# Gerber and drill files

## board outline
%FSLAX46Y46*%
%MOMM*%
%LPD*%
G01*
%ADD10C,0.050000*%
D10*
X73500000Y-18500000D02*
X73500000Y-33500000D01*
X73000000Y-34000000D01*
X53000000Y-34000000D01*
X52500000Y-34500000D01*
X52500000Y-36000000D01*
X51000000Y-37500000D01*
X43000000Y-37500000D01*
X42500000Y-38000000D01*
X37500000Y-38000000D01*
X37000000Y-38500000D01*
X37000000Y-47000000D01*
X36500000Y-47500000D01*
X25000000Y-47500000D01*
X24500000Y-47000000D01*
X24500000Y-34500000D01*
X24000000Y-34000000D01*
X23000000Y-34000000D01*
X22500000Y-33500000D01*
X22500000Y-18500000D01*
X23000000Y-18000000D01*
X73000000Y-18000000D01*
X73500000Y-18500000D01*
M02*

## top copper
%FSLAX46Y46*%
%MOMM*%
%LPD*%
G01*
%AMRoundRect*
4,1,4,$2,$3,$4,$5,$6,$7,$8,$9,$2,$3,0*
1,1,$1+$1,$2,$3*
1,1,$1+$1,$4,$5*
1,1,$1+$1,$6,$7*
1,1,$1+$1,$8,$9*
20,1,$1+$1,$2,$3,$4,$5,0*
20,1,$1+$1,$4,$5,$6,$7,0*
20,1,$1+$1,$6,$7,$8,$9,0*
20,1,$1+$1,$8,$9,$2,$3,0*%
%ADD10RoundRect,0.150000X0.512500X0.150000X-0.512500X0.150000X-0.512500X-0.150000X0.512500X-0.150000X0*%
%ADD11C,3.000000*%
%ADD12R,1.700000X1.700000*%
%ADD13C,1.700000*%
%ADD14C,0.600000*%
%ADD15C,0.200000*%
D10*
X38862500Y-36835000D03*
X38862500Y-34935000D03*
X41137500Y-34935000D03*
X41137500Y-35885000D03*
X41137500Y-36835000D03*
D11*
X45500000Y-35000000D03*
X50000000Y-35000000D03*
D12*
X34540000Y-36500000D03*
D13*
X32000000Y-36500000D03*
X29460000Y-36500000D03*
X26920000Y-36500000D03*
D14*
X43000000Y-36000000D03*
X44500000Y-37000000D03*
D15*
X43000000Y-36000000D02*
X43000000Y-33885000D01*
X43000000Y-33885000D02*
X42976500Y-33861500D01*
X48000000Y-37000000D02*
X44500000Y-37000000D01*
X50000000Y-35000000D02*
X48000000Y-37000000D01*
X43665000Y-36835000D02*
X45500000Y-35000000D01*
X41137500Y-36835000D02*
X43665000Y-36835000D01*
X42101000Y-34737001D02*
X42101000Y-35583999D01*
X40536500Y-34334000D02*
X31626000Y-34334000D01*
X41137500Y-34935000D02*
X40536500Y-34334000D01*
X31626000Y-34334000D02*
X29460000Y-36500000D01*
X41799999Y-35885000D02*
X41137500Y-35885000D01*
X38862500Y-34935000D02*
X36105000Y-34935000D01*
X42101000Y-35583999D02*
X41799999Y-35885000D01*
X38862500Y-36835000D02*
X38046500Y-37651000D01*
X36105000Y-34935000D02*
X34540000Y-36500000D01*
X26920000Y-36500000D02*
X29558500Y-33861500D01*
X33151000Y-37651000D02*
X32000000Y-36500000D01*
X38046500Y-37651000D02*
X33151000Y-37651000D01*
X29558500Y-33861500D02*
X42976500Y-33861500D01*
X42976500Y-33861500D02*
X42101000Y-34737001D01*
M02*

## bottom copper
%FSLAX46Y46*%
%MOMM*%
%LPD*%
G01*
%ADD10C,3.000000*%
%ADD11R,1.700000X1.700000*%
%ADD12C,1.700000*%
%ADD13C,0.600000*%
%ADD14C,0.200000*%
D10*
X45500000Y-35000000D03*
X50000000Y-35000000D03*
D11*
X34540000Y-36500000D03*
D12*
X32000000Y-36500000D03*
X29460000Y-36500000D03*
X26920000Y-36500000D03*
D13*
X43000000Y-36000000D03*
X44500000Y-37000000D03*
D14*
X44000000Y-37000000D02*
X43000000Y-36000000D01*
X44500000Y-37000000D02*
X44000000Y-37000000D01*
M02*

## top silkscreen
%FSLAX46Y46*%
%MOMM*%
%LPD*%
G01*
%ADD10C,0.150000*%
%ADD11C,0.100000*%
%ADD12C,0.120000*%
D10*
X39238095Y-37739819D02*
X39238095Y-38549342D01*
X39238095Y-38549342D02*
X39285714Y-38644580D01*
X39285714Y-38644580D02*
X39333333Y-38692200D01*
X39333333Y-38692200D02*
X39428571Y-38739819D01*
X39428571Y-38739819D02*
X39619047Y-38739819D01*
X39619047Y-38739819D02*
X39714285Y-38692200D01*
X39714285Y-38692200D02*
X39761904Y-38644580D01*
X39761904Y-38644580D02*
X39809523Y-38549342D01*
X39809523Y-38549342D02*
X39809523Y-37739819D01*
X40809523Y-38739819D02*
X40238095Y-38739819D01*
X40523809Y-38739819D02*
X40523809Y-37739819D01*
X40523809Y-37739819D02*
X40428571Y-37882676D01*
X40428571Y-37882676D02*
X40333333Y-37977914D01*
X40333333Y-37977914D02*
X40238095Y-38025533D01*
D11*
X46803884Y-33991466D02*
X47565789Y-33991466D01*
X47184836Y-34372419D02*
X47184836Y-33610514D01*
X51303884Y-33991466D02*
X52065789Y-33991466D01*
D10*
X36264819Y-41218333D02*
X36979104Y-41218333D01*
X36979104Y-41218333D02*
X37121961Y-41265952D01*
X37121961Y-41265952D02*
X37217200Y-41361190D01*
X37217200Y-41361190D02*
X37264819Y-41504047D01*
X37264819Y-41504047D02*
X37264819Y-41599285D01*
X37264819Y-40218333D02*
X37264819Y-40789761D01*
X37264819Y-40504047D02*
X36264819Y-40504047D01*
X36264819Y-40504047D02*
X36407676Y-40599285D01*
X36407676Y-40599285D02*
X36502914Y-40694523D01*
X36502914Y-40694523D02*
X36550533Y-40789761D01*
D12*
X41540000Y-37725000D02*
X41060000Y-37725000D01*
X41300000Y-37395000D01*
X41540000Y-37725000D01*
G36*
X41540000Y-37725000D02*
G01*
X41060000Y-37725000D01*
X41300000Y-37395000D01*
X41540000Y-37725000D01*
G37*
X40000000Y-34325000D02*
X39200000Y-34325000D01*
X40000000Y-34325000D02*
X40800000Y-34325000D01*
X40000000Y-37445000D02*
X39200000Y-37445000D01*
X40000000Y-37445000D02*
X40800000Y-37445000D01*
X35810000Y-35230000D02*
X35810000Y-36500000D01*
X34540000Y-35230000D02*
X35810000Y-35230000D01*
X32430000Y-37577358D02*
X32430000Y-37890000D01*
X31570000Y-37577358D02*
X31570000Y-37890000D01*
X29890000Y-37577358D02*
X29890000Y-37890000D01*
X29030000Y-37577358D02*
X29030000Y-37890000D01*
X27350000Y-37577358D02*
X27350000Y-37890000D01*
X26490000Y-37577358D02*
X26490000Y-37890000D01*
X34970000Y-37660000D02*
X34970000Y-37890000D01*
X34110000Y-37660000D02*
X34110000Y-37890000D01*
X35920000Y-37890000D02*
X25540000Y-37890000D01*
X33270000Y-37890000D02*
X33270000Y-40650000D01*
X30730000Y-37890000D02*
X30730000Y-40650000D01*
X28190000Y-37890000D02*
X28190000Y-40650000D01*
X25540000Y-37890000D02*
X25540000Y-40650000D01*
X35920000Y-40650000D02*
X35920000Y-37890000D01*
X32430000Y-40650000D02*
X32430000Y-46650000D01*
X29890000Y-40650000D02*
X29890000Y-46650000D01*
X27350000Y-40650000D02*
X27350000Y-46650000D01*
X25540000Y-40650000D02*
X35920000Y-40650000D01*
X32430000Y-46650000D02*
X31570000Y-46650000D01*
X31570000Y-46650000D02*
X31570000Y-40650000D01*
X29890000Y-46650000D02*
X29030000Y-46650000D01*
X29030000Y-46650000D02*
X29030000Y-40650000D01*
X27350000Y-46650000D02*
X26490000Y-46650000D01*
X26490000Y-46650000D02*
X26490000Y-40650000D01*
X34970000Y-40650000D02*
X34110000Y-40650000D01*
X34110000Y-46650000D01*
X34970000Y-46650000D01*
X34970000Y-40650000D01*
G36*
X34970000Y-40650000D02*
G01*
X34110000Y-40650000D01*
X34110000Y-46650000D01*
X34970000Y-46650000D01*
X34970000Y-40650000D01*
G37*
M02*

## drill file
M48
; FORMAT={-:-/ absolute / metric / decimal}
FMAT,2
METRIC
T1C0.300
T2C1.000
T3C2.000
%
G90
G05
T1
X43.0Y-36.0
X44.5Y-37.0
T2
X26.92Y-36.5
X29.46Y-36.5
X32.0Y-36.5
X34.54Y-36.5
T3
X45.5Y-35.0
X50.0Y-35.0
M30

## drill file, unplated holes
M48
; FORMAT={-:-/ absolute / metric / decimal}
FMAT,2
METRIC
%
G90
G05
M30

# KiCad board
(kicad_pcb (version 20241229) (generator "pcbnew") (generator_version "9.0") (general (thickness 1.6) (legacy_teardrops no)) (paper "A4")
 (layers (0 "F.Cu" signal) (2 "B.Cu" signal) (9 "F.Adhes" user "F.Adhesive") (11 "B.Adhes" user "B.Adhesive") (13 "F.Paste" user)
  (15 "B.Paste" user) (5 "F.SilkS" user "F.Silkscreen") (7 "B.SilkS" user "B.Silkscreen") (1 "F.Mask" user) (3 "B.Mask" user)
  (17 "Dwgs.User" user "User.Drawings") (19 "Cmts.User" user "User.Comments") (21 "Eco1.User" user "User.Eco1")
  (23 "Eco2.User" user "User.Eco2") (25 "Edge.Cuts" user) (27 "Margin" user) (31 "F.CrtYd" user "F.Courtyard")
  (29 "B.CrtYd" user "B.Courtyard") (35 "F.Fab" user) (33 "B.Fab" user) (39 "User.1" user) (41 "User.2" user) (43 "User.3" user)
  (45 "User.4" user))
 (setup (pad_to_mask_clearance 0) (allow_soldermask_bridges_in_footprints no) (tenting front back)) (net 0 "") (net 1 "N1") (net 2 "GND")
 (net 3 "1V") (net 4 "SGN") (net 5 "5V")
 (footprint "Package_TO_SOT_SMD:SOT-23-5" (layer "F.Cu") (at 40 35.885 180)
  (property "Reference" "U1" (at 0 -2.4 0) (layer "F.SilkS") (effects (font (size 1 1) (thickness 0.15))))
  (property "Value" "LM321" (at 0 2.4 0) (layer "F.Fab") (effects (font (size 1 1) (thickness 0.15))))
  (fp_line (start 0 1.56) (end 0.8 1.56) (stroke (width 0.12) (type solid)) (layer "F.SilkS"))
  (fp_line (start 0 1.56) (end -0.8 1.56) (stroke (width 0.12) (type solid)) (layer "F.SilkS"))
  (fp_line (start 0 -1.56) (end 0.8 -1.56) (stroke (width 0.12) (type solid)) (layer "F.SilkS"))
  (fp_line (start 0 -1.56) (end -0.8 -1.56) (stroke (width 0.12) (type solid)) (layer "F.SilkS"))
  (fp_poly (pts (xy -1.3 -1.51) (xy -1.54 -1.84) (xy -1.06 -1.84)) (stroke (width 0.12) (type solid)) (fill yes) (layer "F.SilkS"))
  (pad "1" smd roundrect (at -1.1375 -0.95 180) (size 1.325 0.6) (layers "F.Cu" "F.Mask" "F.Paste") (roundrect_rratio 0.25) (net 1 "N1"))
  (pad "2" smd roundrect (at -1.1375 0 180) (size 1.325 0.6) (layers "F.Cu" "F.Mask" "F.Paste") (roundrect_rratio 0.25) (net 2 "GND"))
  (pad "3" smd roundrect (at -1.1375 0.95 180) (size 1.325 0.6) (layers "F.Cu" "F.Mask" "F.Paste") (roundrect_rratio 0.25) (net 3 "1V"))
  (pad "4" smd roundrect (at 1.1375 0.95 180) (size 1.325 0.6) (layers "F.Cu" "F.Mask" "F.Paste") (roundrect_rratio 0.25) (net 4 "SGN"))
  (pad "5" smd roundrect (at 1.1375 -0.95 180) (size 1.325 0.6) (layers "F.Cu" "F.Mask" "F.Paste") (roundrect_rratio 0.25) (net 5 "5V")))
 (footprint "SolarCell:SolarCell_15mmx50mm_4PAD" (layer "F.Cu") (at 48 26)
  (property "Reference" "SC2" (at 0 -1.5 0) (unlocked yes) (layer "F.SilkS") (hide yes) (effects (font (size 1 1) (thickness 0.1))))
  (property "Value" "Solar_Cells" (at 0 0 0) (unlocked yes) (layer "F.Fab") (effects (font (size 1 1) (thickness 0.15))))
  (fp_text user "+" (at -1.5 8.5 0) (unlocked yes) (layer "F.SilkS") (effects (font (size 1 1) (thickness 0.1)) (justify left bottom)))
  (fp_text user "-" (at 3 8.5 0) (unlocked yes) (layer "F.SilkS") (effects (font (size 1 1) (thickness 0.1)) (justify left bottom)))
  (pad "1" thru_hole circle (at -2.5 9) (size 3 3) (drill 2) (layers "*.Cu" "*.Mask" "Dwgs.User") (remove_unused_layers no) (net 1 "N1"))
  (pad "2" thru_hole circle (at 2 9) (size 3 3) (drill 2) (layers "*.Cu" "*.Mask" "Dwgs.User") (remove_unused_layers no) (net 2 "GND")))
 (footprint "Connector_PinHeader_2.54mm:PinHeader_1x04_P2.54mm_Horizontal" (layer "F.Cu") (at 34.54 36.5 -90)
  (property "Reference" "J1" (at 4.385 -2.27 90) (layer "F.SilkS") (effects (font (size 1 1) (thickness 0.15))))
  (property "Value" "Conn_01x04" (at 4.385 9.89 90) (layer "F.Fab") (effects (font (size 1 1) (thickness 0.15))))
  (fp_line (start 1.39 9) (end 4.15 9) (stroke (width 0.12) (type solid)) (layer "F.SilkS"))
  (fp_line (start 4.15 9) (end 4.15 -1.38) (stroke (width 0.12) (type solid)) (layer "F.SilkS"))
  (fp_line (start 1.077358 8.05) (end 1.39 8.05) (stroke (width 0.12) (type solid)) (layer "F.SilkS"))
  (fp_line (start 10.15 8.05) (end 4.15 8.05) (stroke (width 0.12) (type solid)) (layer "F.SilkS"))
  (fp_line (start 1.077358 7.19) (end 1.39 7.19) (stroke (width 0.12) (type solid)) (layer "F.SilkS"))
  (fp_line (start 4.15 7.19) (end 10.15 7.19) (stroke (width 0.12) (type solid)) (layer "F.SilkS"))
  (fp_line (start 10.15 7.19) (end 10.15 8.05) (stroke (width 0.12) (type solid)) (layer "F.SilkS"))
  (fp_line (start 1.39 6.35) (end 4.15 6.35) (stroke (width 0.12) (type solid)) (layer "F.SilkS"))
  (fp_line (start 1.077358 5.51) (end 1.39 5.51) (stroke (width 0.12) (type solid)) (layer "F.SilkS"))
  (fp_line (start 10.15 5.51) (end 4.15 5.51) (stroke (width 0.12) (type solid)) (layer "F.SilkS"))
  (fp_line (start 1.077358 4.65) (end 1.39 4.65) (stroke (width 0.12) (type solid)) (layer "F.SilkS"))
  (fp_line (start 4.15 4.65) (end 10.15 4.65) (stroke (width 0.12) (type solid)) (layer "F.SilkS"))
  (fp_line (start 10.15 4.65) (end 10.15 5.51) (stroke (width 0.12) (type solid)) (layer "F.SilkS"))
  (fp_line (start 1.39 3.81) (end 4.15 3.81) (stroke (width 0.12) (type solid)) (layer "F.SilkS"))
  (fp_line (start 1.077358 2.97) (end 1.39 2.97) (stroke (width 0.12) (type solid)) (layer "F.SilkS"))
  (fp_line (start 10.15 2.97) (end 4.15 2.97) (stroke (width 0.12) (type solid)) (layer "F.SilkS"))
  (fp_line (start 1.077358 2.11) (end 1.39 2.11) (stroke (width 0.12) (type solid)) (layer "F.SilkS"))
  (fp_line (start 4.15 2.11) (end 10.15 2.11) (stroke (width 0.12) (type solid)) (layer "F.SilkS"))
  (fp_line (start 10.15 2.11) (end 10.15 2.97) (stroke (width 0.12) (type solid)) (layer "F.SilkS"))
  (fp_line (start 1.39 1.27) (end 4.15 1.27) (stroke (width 0.12) (type solid)) (layer "F.SilkS"))
  (fp_line (start 1.16 0.43) (end 1.39 0.43) (stroke (width 0.12) (type solid)) (layer "F.SilkS"))
  (fp_line (start -1.27 0) (end -1.27 -1.27) (stroke (width 0.12) (type solid)) (layer "F.SilkS"))
  (fp_line (start 1.16 -0.43) (end 1.39 -0.43) (stroke (width 0.12) (type solid)) (layer "F.SilkS"))
  (fp_line (start -1.27 -1.27) (end 0 -1.27) (stroke (width 0.12) (type solid)) (layer "F.SilkS"))
  (fp_line (start 1.39 -1.38) (end 1.39 9) (stroke (width 0.12) (type solid)) (layer "F.SilkS"))
  (fp_line (start 4.15 -1.38) (end 1.39 -1.38) (stroke (width 0.12) (type solid)) (layer "F.SilkS"))
  (fp_rect (start 4.15 -0.43) (end 10.15 0.43) (stroke (width 0.12) (type solid)) (fill yes) (layer "F.SilkS"))
  (pad "1" thru_hole rect (at 0 0 270) (size 1.7 1.7) (drill 1) (layers "*.Cu" "*.Mask") (remove_unused_layers no) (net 4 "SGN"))
  (pad "2" thru_hole circle (at 0 2.54 270) (size 1.7 1.7) (drill 1) (layers "*.Cu" "*.Mask") (remove_unused_layers no) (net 5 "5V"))
  (pad "3" thru_hole circle (at 0 5.08 270) (size 1.7 1.7) (drill 1) (layers "*.Cu" "*.Mask") (remove_unused_layers no) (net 3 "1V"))
  (pad "4" thru_hole circle (at 0 7.62 270) (size 1.7 1.7) (drill 1) (layers "*.Cu" "*.Mask") (remove_unused_layers no) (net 2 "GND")))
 (gr_poly
  (pts (xy 23 18) (xy 22.5 18.5) (xy 22.5 33.5) (xy 23 34) (xy 24 34) (xy 24.5 34.5) (xy 24.5 47) (xy 25 47.5) (xy 36.5 47.5) (xy 37 47)
   (xy 37 38.5) (xy 37.5 38) (xy 42.5 38) (xy 43 37.5) (xy 51 37.5) (xy 52.5 36) (xy 52.5 34.5) (xy 53 34) (xy 73 34) (xy 73.5 33.5)
   (xy 73.5 18.5) (xy 73 18))
  (stroke (width 0.05) (type solid)) (fill no) (layer "Edge.Cuts"))
 (segment (start 41.1375 34.935) (end 40.5365 34.334) (width 0.2) (layer "F.Cu") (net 3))
 (segment (start 31.626 34.334) (end 29.46 36.5) (width 0.2) (layer "F.Cu") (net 3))
 (segment (start 40.5365 34.334) (end 31.626 34.334) (width 0.2) (layer "F.Cu") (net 3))
 (segment (start 36.105 34.935) (end 34.54 36.5) (width 0.2) (layer "F.Cu") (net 4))
 (segment (start 38.8625 34.935) (end 36.105 34.935) (width 0.2) (layer "F.Cu") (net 4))
 (segment (start 38.8625 36.835) (end 38.0465 37.651) (width 0.2) (layer "F.Cu") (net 5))
 (segment (start 38.0465 37.651) (end 33.151 37.651) (width 0.2) (layer "F.Cu") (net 5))
 (segment (start 33.151 37.651) (end 32 36.5) (width 0.2) (layer "F.Cu") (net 5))
 (segment (start 29.5585 33.8615) (end 42.9765 33.8615) (width 0.2) (layer "F.Cu") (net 2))
 (segment (start 50 35) (end 48 37) (width 0.2) (layer "F.Cu") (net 2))
 (segment (start 48 37) (end 44.5 37) (width 0.2) (layer "F.Cu") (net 2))
 (segment (start 41.799999 35.885) (end 41.1375 35.885) (width 0.2) (layer "F.Cu") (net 2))
 (segment (start 42.9765 33.8615) (end 42.101 34.737001) (width 0.2) (layer "F.Cu") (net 2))
 (segment (start 43 33.885) (end 42.9765 33.8615) (width 0.2) (layer "F.Cu") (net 2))
 (segment (start 43 36) (end 43 33.885) (width 0.2) (layer "F.Cu") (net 2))
 (segment (start 26.92 36.5) (end 29.5585 33.8615) (width 0.2) (layer "F.Cu") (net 2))
 (segment (start 42.101 34.737001) (end 42.101 35.583999) (width 0.2) (layer "F.Cu") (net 2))
 (segment (start 42.101 35.583999) (end 41.799999 35.885) (width 0.2) (layer "F.Cu") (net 2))
 (via (at 44.5 37) (size 0.6) (drill 0.3) (layers "F.Cu" "B.Cu") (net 2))
 (via (at 43 36) (size 0.6) (drill 0.3) (layers "F.Cu" "B.Cu") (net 2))
 (segment (start 44 37) (end 43 36) (width 0.2) (layer "B.Cu") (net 2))
 (segment (start 44.5 37) (end 44 37) (width 0.2) (layer "B.Cu") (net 2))
 (segment (start 41.1375 36.835) (end 43.665 36.835) (width 0.2) (layer "F.Cu") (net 1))
 (segment (start 43.665 36.835) (end 45.5 35) (width 0.2) (layer "F.Cu") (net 1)))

